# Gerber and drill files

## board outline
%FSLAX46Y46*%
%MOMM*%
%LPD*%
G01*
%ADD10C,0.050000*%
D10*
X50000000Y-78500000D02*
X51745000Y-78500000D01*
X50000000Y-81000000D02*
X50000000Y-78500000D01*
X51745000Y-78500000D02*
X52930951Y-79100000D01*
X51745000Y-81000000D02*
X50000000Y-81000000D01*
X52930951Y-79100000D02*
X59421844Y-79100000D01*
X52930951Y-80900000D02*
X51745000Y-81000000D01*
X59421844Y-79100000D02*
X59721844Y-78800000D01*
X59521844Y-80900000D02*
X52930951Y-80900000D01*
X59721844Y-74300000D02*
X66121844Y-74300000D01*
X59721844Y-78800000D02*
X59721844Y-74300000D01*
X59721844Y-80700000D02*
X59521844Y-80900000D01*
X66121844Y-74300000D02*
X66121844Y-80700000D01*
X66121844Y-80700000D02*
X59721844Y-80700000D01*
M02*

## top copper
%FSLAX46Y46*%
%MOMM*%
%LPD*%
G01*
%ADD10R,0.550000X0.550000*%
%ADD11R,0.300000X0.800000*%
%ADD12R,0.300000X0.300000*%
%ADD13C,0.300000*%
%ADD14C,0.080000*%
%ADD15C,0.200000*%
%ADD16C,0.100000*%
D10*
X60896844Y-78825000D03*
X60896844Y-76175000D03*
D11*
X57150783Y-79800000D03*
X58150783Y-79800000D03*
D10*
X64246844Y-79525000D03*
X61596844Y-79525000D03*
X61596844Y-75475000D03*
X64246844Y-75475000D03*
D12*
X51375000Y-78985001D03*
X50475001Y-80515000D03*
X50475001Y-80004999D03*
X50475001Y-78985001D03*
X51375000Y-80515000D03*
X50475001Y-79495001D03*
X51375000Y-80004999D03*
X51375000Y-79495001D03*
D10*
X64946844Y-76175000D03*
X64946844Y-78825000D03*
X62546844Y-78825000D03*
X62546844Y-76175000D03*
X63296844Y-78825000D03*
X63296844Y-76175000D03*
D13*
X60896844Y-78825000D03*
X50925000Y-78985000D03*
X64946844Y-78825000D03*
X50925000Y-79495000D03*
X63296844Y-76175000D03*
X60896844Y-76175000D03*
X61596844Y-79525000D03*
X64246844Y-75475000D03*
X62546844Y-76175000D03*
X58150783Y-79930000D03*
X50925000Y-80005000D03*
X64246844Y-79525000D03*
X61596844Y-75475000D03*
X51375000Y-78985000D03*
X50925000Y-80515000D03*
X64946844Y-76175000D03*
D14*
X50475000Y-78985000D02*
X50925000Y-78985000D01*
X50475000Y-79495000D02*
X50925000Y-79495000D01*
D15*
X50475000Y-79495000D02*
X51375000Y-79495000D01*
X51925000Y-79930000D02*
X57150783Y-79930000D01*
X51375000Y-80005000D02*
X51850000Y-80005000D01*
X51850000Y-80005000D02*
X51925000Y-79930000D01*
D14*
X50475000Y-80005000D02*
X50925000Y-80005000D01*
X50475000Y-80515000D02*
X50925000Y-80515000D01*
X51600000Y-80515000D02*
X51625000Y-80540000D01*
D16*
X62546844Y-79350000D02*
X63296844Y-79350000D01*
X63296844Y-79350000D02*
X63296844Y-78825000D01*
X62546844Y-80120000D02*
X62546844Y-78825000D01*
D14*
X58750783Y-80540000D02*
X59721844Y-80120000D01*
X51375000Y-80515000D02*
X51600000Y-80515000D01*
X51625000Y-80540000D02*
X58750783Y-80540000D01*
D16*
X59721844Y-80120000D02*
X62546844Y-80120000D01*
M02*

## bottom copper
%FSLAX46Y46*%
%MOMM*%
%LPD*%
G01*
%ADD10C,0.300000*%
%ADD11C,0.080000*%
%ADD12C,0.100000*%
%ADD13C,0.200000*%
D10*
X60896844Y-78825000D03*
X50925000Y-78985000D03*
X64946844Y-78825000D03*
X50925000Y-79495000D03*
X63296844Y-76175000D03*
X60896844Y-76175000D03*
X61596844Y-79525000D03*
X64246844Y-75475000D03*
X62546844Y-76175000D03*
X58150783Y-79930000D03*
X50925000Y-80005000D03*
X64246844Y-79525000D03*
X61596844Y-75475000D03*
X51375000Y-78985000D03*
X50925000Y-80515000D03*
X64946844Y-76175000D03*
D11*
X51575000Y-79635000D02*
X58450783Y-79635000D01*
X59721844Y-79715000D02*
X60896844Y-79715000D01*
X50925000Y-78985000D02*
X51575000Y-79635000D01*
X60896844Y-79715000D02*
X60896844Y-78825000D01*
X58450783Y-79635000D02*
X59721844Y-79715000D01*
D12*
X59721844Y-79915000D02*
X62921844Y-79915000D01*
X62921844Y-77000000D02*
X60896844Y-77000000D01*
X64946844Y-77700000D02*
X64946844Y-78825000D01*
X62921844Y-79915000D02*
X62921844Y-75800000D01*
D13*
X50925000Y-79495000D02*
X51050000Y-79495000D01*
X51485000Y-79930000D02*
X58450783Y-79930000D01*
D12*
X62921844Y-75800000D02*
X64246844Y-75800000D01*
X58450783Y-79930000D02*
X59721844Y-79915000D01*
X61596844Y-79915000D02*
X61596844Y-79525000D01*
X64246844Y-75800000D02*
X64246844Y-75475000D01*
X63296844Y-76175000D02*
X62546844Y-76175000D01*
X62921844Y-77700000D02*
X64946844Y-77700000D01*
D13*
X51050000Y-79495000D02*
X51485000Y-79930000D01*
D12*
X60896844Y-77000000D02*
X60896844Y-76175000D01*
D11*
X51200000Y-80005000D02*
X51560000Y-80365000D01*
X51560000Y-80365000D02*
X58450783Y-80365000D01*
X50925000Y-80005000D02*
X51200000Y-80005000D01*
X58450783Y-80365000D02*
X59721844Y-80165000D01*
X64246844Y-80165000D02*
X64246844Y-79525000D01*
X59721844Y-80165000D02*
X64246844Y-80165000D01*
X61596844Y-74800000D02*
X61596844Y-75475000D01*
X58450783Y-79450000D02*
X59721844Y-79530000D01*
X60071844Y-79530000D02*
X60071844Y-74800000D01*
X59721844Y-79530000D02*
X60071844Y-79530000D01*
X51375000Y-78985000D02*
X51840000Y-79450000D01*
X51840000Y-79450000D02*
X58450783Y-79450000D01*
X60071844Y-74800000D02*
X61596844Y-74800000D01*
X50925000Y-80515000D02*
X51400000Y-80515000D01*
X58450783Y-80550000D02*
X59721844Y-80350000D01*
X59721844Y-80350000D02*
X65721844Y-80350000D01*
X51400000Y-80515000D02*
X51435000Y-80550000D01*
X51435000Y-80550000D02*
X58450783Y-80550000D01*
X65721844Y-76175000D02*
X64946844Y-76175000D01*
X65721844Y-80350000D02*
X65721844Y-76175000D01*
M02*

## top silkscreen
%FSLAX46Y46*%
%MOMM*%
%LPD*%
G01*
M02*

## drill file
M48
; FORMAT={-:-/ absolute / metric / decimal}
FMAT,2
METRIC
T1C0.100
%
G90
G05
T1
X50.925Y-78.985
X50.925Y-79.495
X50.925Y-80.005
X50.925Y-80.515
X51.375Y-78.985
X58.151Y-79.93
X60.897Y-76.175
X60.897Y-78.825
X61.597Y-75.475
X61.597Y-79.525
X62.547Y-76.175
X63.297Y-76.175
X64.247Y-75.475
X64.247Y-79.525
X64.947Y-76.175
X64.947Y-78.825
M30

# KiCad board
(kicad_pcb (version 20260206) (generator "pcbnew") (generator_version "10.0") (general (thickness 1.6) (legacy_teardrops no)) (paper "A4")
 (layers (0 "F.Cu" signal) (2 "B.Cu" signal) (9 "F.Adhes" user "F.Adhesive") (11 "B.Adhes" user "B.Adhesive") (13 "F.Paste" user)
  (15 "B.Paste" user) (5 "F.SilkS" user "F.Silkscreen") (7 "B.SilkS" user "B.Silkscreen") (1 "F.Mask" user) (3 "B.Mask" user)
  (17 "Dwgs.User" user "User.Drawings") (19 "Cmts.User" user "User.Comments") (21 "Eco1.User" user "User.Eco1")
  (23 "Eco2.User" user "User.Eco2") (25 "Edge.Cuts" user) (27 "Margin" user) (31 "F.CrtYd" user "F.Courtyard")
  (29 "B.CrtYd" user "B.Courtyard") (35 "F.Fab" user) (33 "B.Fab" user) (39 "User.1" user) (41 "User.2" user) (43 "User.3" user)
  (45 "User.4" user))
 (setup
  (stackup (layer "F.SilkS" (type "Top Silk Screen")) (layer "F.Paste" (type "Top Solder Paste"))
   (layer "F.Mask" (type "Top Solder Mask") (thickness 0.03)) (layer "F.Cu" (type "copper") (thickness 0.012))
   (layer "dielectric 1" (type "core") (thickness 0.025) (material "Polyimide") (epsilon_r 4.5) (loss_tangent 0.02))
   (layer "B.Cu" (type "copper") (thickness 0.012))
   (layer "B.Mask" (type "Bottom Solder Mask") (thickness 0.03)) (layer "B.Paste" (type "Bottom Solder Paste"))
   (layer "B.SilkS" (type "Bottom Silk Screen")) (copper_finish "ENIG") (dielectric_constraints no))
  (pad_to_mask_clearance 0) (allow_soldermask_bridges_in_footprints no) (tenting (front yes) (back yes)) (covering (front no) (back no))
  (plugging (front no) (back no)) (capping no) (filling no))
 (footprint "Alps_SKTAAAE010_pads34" (layer "F.Cu") (at 60.521844 77.5 90)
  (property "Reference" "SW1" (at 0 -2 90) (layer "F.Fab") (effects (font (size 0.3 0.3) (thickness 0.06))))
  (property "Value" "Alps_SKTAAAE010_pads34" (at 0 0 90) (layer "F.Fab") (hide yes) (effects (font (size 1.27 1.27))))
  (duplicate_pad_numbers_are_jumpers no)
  (pad "3" smd rect (at -1.325 0.375 90) (size 0.55 0.55) (layers "F.Cu" "F.Mask") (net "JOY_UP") (solder_mask_margin 0.05)
   (thermal_bridge_angle 45))
  (pad "4" smd rect (at 1.325 0.375 90) (size 0.55 0.55) (layers "F.Cu" "F.Mask") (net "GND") (solder_mask_margin 0.05)
   (thermal_bridge_angle 45)))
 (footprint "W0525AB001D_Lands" (layer "F.Cu") (at 57.650783 79.93)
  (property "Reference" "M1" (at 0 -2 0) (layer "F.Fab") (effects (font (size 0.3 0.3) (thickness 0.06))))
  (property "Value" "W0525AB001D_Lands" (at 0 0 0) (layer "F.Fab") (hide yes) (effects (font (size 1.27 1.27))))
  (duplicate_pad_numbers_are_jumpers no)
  (pad "1" smd rect (at -0.5 -0.13) (size 0.3 0.8) (layers "F.Cu" "F.Mask") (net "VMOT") (solder_mask_margin 0.05) (thermal_bridge_angle 45))
  (pad "2" smd rect (at 0.5 -0.13) (size 0.3 0.8) (layers "F.Cu" "F.Mask") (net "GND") (solder_mask_margin 0.05) (thermal_bridge_angle 45)))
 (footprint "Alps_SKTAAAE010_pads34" (layer "F.Cu") (at 62.921844 79.9 180)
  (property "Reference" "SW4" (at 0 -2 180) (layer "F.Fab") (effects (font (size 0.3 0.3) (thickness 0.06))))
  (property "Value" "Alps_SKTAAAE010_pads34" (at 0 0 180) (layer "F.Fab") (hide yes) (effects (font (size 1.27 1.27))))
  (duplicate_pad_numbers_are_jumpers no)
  (pad "3" smd rect (at -1.325 0.375 180) (size 0.55 0.55) (layers "F.Cu" "F.Mask") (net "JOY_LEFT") (solder_mask_margin 0.05)
   (thermal_bridge_angle 45))
  (pad "4" smd rect (at 1.325 0.375 180) (size 0.55 0.55) (layers "F.Cu" "F.Mask") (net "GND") (solder_mask_margin 0.05)
   (thermal_bridge_angle 45)))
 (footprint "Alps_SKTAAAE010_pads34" (layer "F.Cu") (at 62.921844 75.1)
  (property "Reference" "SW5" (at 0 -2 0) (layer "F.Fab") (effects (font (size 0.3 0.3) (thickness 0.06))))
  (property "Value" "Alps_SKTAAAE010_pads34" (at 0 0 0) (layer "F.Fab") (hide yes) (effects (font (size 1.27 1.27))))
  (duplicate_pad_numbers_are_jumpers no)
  (pad "3" smd rect (at -1.325 0.375) (size 0.55 0.55) (layers "F.Cu" "F.Mask") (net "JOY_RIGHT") (solder_mask_margin 0.05)
   (thermal_bridge_angle 45))
  (pad "4" smd rect (at 1.325 0.375) (size 0.55 0.55) (layers "F.Cu" "F.Mask") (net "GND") (solder_mask_margin 0.05)
   (thermal_bridge_angle 45)))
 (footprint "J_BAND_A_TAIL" (layer "F.Cu") (at 50.9 79.75)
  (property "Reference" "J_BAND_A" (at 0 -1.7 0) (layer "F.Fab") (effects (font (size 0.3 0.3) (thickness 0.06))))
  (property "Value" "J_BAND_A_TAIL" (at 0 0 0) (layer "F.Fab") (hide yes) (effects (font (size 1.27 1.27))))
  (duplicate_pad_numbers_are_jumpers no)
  (pad "1" smd rect (at 0.475 -0.764999) (size 0.3 0.3) (layers "F.Cu" "F.Mask") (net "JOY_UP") (solder_mask_margin 0.05)
   (thermal_bridge_angle 45))
  (pad "2" smd rect (at -0.424999 0.765) (size 0.3 0.3) (layers "F.Cu" "F.Mask") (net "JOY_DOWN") (solder_mask_margin 0.05)
   (thermal_bridge_angle 45))
  (pad "3" smd rect (at -0.424999 0.254999) (size 0.3 0.3) (layers "F.Cu" "F.Mask") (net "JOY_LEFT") (solder_mask_margin 0.05)
   (thermal_bridge_angle 45))
  (pad "4" smd rect (at -0.424999 -0.764999) (size 0.3 0.3) (layers "F.Cu" "F.Mask") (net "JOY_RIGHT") (solder_mask_margin 0.05)
   (thermal_bridge_angle 45))
  (pad "5" smd rect (at 0.475 0.765) (size 0.3 0.3) (layers "F.Cu" "F.Mask") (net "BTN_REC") (solder_mask_margin 0.05)
   (thermal_bridge_angle 45))
  (pad "6" smd rect (at -0.424999 -0.254999) (size 0.3 0.3) (layers "F.Cu" "F.Mask") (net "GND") (solder_mask_margin 0.05)
   (thermal_bridge_angle 45))
  (pad "7" smd rect (at 0.475 0.254999) (size 0.3 0.3) (layers "F.Cu" "F.Mask") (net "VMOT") (solder_mask_margin 0.05)
   (thermal_bridge_angle 45))
  (pad "8" smd rect (at 0.475 -0.254999) (size 0.3 0.3) (layers "F.Cu" "F.Mask") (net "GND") (solder_mask_margin 0.05)
   (thermal_bridge_angle 45)))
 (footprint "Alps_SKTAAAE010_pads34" (layer "F.Cu") (at 65.321844 77.5 -90)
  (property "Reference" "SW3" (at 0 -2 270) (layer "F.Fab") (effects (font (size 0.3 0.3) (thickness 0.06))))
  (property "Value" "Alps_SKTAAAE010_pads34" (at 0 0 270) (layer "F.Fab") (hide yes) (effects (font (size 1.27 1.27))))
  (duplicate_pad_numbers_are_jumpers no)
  (pad "3" smd rect (at -1.325 0.375 270) (size 0.55 0.55) (layers "F.Cu" "F.Mask") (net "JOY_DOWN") (solder_mask_margin 0.05)
   (thermal_bridge_angle 45))
  (pad "4" smd rect (at 1.325 0.375 270) (size 0.55 0.55) (layers "F.Cu" "F.Mask") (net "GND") (solder_mask_margin 0.05)
   (thermal_bridge_angle 45)))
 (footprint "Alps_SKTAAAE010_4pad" (layer "F.Cu") (at 62.921844 77.5 90)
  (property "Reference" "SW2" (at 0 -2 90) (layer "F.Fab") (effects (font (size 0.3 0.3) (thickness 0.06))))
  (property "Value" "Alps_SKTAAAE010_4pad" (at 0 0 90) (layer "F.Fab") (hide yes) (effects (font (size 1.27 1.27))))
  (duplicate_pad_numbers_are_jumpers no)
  (pad "1" smd rect (at -1.325 -0.375 90) (size 0.55 0.55) (layers "F.Cu" "F.Mask") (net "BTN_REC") (solder_mask_margin 0.05)
   (thermal_bridge_angle 45))
  (pad "2" smd rect (at 1.325 -0.375 90) (size 0.55 0.55) (layers "F.Cu" "F.Mask") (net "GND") (solder_mask_margin 0.05)
   (thermal_bridge_angle 45))
  (pad "3" smd rect (at -1.325 0.375 90) (size 0.55 0.55) (layers "F.Cu" "F.Mask") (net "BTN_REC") (solder_mask_margin 0.05)
   (thermal_bridge_angle 45))
  (pad "4" smd rect (at 1.325 0.375 90) (size 0.55 0.55) (layers "F.Cu" "F.Mask") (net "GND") (solder_mask_margin 0.05)
   (thermal_bridge_angle 45)))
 (gr_line (start 50 78.5) (end 51.745 78.5) (stroke (width 0.05) (type default)) (layer "Edge.Cuts"))
 (gr_line (start 50 81) (end 50 78.5) (stroke (width 0.05) (type default)) (layer "Edge.Cuts"))
 (gr_line (start 51.745 78.5) (end 52.930951 79.1) (stroke (width 0.05) (type default)) (layer "Edge.Cuts"))
 (gr_line (start 51.745 81) (end 50 81) (stroke (width 0.05) (type default)) (layer "Edge.Cuts"))
 (gr_line (start 52.930951 79.1) (end 59.421844 79.1) (stroke (width 0.05) (type default)) (layer "Edge.Cuts"))
 (gr_line (start 52.930951 80.9) (end 51.745 81) (stroke (width 0.05) (type default)) (layer "Edge.Cuts"))
 (gr_line (start 59.421844 79.1) (end 59.721844 78.8) (stroke (width 0.05) (type default)) (layer "Edge.Cuts"))
 (gr_line (start 59.521844 80.9) (end 52.930951 80.9) (stroke (width 0.05) (type default)) (layer "Edge.Cuts"))
 (gr_line (start 59.721844 74.3) (end 66.121844 74.3) (stroke (width 0.05) (type default)) (layer "Edge.Cuts"))
 (gr_line (start 59.721844 78.8) (end 59.721844 74.3) (stroke (width 0.05) (type default)) (layer "Edge.Cuts"))
 (gr_line (start 59.721844 80.7) (end 59.521844 80.9) (stroke (width 0.05) (type default)) (layer "Edge.Cuts"))
 (gr_line (start 66.121844 74.3) (end 66.121844 80.7) (stroke (width 0.05) (type default)) (layer "Edge.Cuts"))
 (gr_line (start 66.121844 80.7) (end 59.721844 80.7) (stroke (width 0.05) (type default)) (layer "Edge.Cuts"))
 (segment (start 50.475 78.985) (end 50.925 78.985) (width 0.08) (layer "F.Cu") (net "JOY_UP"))
 (via (at 60.896844 78.825) (size 0.3) (drill 0.1) (layers "F.Cu" "B.Cu") (tenting (front yes) (back yes)) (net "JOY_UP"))
 (via (at 50.925 78.985) (size 0.3) (drill 0.1) (layers "F.Cu" "B.Cu") (tenting (front yes) (back yes)) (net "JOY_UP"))
 (segment (start 51.575 79.635) (end 58.450783 79.635) (width 0.08) (layer "B.Cu") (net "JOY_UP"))
 (segment (start 59.721844 79.715) (end 60.896844 79.715) (width 0.08) (layer "B.Cu") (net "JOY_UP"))
 (segment (start 50.925 78.985) (end 51.575 79.635) (width 0.08) (layer "B.Cu") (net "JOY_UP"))
 (segment (start 60.896844 79.715) (end 60.896844 78.825) (width 0.08) (layer "B.Cu") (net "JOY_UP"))
 (segment (start 58.450783 79.635) (end 59.721844 79.715) (width 0.08) (layer "B.Cu") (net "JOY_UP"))
 (segment (start 50.475 79.495) (end 50.925 79.495) (width 0.08) (layer "F.Cu") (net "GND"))
 (segment (start 50.475 79.495) (end 51.375 79.495) (width 0.2) (layer "F.Cu") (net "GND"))
 (via (at 64.946844 78.825) (size 0.3) (drill 0.1) (layers "F.Cu" "B.Cu") (tenting (front yes) (back yes)) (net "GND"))
 (via (at 50.925 79.495) (size 0.3) (drill 0.1) (layers "F.Cu" "B.Cu") (tenting (front yes) (back yes)) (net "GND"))
 (via (at 63.296844 76.175) (size 0.3) (drill 0.1) (layers "F.Cu" "B.Cu") (tenting (front yes) (back yes)) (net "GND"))
 (via (at 60.896844 76.175) (size 0.3) (drill 0.1) (layers "F.Cu" "B.Cu") (tenting (front yes) (back yes)) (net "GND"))
 (via (at 61.596844 79.525) (size 0.3) (drill 0.1) (layers "F.Cu" "B.Cu") (tenting (front yes) (back yes)) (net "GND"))
 (via (at 64.246844 75.475) (size 0.3) (drill 0.1) (layers "F.Cu" "B.Cu") (tenting (front yes) (back yes)) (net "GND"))
 (via (at 62.546844 76.175) (size 0.3) (drill 0.1) (layers "F.Cu" "B.Cu") (tenting (front yes) (back yes)) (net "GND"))
 (via (at 58.150783 79.93) (size 0.3) (drill 0.1) (layers "F.Cu" "B.Cu") (tenting (front yes) (back yes)) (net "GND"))
 (segment (start 59.721844 79.915) (end 62.921844 79.915) (width 0.1) (layer "B.Cu") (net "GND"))
 (segment (start 62.921844 77) (end 60.896844 77) (width 0.1) (layer "B.Cu") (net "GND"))
 (segment (start 64.946844 77.7) (end 64.946844 78.825) (width 0.1) (layer "B.Cu") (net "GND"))
 (segment (start 62.921844 79.915) (end 62.921844 75.8) (width 0.1) (layer "B.Cu") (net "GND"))
 (segment (start 50.925 79.495) (end 51.05 79.495) (width 0.2) (layer "B.Cu") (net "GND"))
 (segment (start 51.485 79.93) (end 58.450783 79.93) (width 0.2) (layer "B.Cu") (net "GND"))
 (segment (start 62.921844 75.8) (end 64.246844 75.8) (width 0.1) (layer "B.Cu") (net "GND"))
 (segment (start 58.450783 79.93) (end 59.721844 79.915) (width 0.1) (layer "B.Cu") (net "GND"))
 (segment (start 61.596844 79.915) (end 61.596844 79.525) (width 0.1) (layer "B.Cu") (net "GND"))
 (segment (start 64.246844 75.8) (end 64.246844 75.475) (width 0.1) (layer "B.Cu") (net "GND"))
 (segment (start 63.296844 76.175) (end 62.546844 76.175) (width 0.1) (layer "B.Cu") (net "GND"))
 (segment (start 62.921844 77.7) (end 64.946844 77.7) (width 0.1) (layer "B.Cu") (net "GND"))
 (segment (start 51.05 79.495) (end 51.485 79.93) (width 0.2) (layer "B.Cu") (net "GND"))
 (segment (start 60.896844 77) (end 60.896844 76.175) (width 0.1) (layer "B.Cu") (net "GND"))
 (segment (start 51.925 79.93) (end 57.150783 79.93) (width 0.2) (layer "F.Cu") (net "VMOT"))
 (segment (start 51.375 80.005) (end 51.85 80.005) (width 0.2) (layer "F.Cu") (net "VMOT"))
 (segment (start 51.85 80.005) (end 51.925 79.93) (width 0.2) (layer "F.Cu") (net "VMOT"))
 (segment (start 50.475 80.005) (end 50.925 80.005) (width 0.08) (layer "F.Cu") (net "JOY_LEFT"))
 (via (at 50.925 80.005) (size 0.3) (drill 0.1) (layers "F.Cu" "B.Cu") (tenting (front yes) (back yes)) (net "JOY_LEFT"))
 (via (at 64.246844 79.525) (size 0.3) (drill 0.1) (layers "F.Cu" "B.Cu") (tenting (front yes) (back yes)) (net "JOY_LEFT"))
 (segment (start 51.2 80.005) (end 51.56 80.365) (width 0.08) (layer "B.Cu") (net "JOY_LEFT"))
 (segment (start 51.56 80.365) (end 58.450783 80.365) (width 0.08) (layer "B.Cu") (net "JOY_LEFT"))
 (segment (start 50.925 80.005) (end 51.2 80.005) (width 0.08) (layer "B.Cu") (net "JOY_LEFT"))
 (segment (start 58.450783 80.365) (end 59.721844 80.165) (width 0.08) (layer "B.Cu") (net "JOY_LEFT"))
 (segment (start 64.246844 80.165) (end 64.246844 79.525) (width 0.08) (layer "B.Cu") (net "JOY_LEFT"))
 (segment (start 59.721844 80.165) (end 64.246844 80.165) (width 0.08) (layer "B.Cu") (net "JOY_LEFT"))
 (via (at 61.596844 75.475) (size 0.3) (drill 0.1) (layers "F.Cu" "B.Cu") (tenting (front yes) (back yes)) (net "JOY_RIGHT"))
 (via (at 51.375 78.985) (size 0.3) (drill 0.1) (layers "F.Cu" "B.Cu") (tenting (front yes) (back yes)) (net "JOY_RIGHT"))
 (segment (start 61.596844 74.8) (end 61.596844 75.475) (width 0.08) (layer "B.Cu") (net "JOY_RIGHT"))
 (segment (start 58.450783 79.45) (end 59.721844 79.53) (width 0.08) (layer "B.Cu") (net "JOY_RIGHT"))
 (segment (start 60.071844 79.53) (end 60.071844 74.8) (width 0.08) (layer "B.Cu") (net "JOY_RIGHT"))
 (segment (start 59.721844 79.53) (end 60.071844 79.53) (width 0.08) (layer "B.Cu") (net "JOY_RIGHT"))
 (segment (start 51.375 78.985) (end 51.84 79.45) (width 0.08) (layer "B.Cu") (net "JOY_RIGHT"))
 (segment (start 51.84 79.45) (end 58.450783 79.45) (width 0.08) (layer "B.Cu") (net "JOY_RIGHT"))
 (segment (start 60.071844 74.8) (end 61.596844 74.8) (width 0.08) (layer "B.Cu") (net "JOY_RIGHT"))
 (segment (start 50.475 80.515) (end 50.925 80.515) (width 0.08) (layer "F.Cu") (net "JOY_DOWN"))
 (via (at 50.925 80.515) (size 0.3) (drill 0.1) (layers "F.Cu" "B.Cu") (tenting (front yes) (back yes)) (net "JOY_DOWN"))
 (via (at 64.946844 76.175) (size 0.3) (drill 0.1) (layers "F.Cu" "B.Cu") (tenting (front yes) (back yes)) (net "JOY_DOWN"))
 (segment (start 50.925 80.515) (end 51.4 80.515) (width 0.08) (layer "B.Cu") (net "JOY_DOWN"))
 (segment (start 58.450783 80.55) (end 59.721844 80.35) (width 0.08) (layer "B.Cu") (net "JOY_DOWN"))
 (segment (start 59.721844 80.35) (end 65.721844 80.35) (width 0.08) (layer "B.Cu") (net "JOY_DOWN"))
 (segment (start 51.4 80.515) (end 51.435 80.55) (width 0.08) (layer "B.Cu") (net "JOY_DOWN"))
 (segment (start 51.435 80.55) (end 58.450783 80.55) (width 0.08) (layer "B.Cu") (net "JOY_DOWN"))
 (segment (start 65.721844 76.175) (end 64.946844 76.175) (width 0.08) (layer "B.Cu") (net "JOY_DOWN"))
 (segment (start 65.721844 80.35) (end 65.721844 76.175) (width 0.08) (layer "B.Cu") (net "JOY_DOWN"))
 (segment (start 51.6 80.515) (end 51.625 80.54) (width 0.08) (layer "F.Cu") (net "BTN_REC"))
 (segment (start 62.546844 79.35) (end 63.296844 79.35) (width 0.1) (layer "F.Cu") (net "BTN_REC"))
 (segment (start 63.296844 79.35) (end 63.296844 78.825) (width 0.1) (layer "F.Cu") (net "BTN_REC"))
 (segment (start 62.546844 80.12) (end 62.546844 78.825) (width 0.1) (layer "F.Cu") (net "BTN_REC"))
 (segment (start 58.750783 80.54) (end 59.721844 80.12) (width 0.08) (layer "F.Cu") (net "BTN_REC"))
 (segment (start 51.375 80.515) (end 51.6 80.515) (width 0.08) (layer "F.Cu") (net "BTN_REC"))
 (segment (start 51.625 80.54) (end 58.750783 80.54) (width 0.08) (layer "F.Cu") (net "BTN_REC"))
 (segment (start 59.721844 80.12) (end 62.546844 80.12) (width 0.1) (layer "F.Cu") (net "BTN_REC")))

